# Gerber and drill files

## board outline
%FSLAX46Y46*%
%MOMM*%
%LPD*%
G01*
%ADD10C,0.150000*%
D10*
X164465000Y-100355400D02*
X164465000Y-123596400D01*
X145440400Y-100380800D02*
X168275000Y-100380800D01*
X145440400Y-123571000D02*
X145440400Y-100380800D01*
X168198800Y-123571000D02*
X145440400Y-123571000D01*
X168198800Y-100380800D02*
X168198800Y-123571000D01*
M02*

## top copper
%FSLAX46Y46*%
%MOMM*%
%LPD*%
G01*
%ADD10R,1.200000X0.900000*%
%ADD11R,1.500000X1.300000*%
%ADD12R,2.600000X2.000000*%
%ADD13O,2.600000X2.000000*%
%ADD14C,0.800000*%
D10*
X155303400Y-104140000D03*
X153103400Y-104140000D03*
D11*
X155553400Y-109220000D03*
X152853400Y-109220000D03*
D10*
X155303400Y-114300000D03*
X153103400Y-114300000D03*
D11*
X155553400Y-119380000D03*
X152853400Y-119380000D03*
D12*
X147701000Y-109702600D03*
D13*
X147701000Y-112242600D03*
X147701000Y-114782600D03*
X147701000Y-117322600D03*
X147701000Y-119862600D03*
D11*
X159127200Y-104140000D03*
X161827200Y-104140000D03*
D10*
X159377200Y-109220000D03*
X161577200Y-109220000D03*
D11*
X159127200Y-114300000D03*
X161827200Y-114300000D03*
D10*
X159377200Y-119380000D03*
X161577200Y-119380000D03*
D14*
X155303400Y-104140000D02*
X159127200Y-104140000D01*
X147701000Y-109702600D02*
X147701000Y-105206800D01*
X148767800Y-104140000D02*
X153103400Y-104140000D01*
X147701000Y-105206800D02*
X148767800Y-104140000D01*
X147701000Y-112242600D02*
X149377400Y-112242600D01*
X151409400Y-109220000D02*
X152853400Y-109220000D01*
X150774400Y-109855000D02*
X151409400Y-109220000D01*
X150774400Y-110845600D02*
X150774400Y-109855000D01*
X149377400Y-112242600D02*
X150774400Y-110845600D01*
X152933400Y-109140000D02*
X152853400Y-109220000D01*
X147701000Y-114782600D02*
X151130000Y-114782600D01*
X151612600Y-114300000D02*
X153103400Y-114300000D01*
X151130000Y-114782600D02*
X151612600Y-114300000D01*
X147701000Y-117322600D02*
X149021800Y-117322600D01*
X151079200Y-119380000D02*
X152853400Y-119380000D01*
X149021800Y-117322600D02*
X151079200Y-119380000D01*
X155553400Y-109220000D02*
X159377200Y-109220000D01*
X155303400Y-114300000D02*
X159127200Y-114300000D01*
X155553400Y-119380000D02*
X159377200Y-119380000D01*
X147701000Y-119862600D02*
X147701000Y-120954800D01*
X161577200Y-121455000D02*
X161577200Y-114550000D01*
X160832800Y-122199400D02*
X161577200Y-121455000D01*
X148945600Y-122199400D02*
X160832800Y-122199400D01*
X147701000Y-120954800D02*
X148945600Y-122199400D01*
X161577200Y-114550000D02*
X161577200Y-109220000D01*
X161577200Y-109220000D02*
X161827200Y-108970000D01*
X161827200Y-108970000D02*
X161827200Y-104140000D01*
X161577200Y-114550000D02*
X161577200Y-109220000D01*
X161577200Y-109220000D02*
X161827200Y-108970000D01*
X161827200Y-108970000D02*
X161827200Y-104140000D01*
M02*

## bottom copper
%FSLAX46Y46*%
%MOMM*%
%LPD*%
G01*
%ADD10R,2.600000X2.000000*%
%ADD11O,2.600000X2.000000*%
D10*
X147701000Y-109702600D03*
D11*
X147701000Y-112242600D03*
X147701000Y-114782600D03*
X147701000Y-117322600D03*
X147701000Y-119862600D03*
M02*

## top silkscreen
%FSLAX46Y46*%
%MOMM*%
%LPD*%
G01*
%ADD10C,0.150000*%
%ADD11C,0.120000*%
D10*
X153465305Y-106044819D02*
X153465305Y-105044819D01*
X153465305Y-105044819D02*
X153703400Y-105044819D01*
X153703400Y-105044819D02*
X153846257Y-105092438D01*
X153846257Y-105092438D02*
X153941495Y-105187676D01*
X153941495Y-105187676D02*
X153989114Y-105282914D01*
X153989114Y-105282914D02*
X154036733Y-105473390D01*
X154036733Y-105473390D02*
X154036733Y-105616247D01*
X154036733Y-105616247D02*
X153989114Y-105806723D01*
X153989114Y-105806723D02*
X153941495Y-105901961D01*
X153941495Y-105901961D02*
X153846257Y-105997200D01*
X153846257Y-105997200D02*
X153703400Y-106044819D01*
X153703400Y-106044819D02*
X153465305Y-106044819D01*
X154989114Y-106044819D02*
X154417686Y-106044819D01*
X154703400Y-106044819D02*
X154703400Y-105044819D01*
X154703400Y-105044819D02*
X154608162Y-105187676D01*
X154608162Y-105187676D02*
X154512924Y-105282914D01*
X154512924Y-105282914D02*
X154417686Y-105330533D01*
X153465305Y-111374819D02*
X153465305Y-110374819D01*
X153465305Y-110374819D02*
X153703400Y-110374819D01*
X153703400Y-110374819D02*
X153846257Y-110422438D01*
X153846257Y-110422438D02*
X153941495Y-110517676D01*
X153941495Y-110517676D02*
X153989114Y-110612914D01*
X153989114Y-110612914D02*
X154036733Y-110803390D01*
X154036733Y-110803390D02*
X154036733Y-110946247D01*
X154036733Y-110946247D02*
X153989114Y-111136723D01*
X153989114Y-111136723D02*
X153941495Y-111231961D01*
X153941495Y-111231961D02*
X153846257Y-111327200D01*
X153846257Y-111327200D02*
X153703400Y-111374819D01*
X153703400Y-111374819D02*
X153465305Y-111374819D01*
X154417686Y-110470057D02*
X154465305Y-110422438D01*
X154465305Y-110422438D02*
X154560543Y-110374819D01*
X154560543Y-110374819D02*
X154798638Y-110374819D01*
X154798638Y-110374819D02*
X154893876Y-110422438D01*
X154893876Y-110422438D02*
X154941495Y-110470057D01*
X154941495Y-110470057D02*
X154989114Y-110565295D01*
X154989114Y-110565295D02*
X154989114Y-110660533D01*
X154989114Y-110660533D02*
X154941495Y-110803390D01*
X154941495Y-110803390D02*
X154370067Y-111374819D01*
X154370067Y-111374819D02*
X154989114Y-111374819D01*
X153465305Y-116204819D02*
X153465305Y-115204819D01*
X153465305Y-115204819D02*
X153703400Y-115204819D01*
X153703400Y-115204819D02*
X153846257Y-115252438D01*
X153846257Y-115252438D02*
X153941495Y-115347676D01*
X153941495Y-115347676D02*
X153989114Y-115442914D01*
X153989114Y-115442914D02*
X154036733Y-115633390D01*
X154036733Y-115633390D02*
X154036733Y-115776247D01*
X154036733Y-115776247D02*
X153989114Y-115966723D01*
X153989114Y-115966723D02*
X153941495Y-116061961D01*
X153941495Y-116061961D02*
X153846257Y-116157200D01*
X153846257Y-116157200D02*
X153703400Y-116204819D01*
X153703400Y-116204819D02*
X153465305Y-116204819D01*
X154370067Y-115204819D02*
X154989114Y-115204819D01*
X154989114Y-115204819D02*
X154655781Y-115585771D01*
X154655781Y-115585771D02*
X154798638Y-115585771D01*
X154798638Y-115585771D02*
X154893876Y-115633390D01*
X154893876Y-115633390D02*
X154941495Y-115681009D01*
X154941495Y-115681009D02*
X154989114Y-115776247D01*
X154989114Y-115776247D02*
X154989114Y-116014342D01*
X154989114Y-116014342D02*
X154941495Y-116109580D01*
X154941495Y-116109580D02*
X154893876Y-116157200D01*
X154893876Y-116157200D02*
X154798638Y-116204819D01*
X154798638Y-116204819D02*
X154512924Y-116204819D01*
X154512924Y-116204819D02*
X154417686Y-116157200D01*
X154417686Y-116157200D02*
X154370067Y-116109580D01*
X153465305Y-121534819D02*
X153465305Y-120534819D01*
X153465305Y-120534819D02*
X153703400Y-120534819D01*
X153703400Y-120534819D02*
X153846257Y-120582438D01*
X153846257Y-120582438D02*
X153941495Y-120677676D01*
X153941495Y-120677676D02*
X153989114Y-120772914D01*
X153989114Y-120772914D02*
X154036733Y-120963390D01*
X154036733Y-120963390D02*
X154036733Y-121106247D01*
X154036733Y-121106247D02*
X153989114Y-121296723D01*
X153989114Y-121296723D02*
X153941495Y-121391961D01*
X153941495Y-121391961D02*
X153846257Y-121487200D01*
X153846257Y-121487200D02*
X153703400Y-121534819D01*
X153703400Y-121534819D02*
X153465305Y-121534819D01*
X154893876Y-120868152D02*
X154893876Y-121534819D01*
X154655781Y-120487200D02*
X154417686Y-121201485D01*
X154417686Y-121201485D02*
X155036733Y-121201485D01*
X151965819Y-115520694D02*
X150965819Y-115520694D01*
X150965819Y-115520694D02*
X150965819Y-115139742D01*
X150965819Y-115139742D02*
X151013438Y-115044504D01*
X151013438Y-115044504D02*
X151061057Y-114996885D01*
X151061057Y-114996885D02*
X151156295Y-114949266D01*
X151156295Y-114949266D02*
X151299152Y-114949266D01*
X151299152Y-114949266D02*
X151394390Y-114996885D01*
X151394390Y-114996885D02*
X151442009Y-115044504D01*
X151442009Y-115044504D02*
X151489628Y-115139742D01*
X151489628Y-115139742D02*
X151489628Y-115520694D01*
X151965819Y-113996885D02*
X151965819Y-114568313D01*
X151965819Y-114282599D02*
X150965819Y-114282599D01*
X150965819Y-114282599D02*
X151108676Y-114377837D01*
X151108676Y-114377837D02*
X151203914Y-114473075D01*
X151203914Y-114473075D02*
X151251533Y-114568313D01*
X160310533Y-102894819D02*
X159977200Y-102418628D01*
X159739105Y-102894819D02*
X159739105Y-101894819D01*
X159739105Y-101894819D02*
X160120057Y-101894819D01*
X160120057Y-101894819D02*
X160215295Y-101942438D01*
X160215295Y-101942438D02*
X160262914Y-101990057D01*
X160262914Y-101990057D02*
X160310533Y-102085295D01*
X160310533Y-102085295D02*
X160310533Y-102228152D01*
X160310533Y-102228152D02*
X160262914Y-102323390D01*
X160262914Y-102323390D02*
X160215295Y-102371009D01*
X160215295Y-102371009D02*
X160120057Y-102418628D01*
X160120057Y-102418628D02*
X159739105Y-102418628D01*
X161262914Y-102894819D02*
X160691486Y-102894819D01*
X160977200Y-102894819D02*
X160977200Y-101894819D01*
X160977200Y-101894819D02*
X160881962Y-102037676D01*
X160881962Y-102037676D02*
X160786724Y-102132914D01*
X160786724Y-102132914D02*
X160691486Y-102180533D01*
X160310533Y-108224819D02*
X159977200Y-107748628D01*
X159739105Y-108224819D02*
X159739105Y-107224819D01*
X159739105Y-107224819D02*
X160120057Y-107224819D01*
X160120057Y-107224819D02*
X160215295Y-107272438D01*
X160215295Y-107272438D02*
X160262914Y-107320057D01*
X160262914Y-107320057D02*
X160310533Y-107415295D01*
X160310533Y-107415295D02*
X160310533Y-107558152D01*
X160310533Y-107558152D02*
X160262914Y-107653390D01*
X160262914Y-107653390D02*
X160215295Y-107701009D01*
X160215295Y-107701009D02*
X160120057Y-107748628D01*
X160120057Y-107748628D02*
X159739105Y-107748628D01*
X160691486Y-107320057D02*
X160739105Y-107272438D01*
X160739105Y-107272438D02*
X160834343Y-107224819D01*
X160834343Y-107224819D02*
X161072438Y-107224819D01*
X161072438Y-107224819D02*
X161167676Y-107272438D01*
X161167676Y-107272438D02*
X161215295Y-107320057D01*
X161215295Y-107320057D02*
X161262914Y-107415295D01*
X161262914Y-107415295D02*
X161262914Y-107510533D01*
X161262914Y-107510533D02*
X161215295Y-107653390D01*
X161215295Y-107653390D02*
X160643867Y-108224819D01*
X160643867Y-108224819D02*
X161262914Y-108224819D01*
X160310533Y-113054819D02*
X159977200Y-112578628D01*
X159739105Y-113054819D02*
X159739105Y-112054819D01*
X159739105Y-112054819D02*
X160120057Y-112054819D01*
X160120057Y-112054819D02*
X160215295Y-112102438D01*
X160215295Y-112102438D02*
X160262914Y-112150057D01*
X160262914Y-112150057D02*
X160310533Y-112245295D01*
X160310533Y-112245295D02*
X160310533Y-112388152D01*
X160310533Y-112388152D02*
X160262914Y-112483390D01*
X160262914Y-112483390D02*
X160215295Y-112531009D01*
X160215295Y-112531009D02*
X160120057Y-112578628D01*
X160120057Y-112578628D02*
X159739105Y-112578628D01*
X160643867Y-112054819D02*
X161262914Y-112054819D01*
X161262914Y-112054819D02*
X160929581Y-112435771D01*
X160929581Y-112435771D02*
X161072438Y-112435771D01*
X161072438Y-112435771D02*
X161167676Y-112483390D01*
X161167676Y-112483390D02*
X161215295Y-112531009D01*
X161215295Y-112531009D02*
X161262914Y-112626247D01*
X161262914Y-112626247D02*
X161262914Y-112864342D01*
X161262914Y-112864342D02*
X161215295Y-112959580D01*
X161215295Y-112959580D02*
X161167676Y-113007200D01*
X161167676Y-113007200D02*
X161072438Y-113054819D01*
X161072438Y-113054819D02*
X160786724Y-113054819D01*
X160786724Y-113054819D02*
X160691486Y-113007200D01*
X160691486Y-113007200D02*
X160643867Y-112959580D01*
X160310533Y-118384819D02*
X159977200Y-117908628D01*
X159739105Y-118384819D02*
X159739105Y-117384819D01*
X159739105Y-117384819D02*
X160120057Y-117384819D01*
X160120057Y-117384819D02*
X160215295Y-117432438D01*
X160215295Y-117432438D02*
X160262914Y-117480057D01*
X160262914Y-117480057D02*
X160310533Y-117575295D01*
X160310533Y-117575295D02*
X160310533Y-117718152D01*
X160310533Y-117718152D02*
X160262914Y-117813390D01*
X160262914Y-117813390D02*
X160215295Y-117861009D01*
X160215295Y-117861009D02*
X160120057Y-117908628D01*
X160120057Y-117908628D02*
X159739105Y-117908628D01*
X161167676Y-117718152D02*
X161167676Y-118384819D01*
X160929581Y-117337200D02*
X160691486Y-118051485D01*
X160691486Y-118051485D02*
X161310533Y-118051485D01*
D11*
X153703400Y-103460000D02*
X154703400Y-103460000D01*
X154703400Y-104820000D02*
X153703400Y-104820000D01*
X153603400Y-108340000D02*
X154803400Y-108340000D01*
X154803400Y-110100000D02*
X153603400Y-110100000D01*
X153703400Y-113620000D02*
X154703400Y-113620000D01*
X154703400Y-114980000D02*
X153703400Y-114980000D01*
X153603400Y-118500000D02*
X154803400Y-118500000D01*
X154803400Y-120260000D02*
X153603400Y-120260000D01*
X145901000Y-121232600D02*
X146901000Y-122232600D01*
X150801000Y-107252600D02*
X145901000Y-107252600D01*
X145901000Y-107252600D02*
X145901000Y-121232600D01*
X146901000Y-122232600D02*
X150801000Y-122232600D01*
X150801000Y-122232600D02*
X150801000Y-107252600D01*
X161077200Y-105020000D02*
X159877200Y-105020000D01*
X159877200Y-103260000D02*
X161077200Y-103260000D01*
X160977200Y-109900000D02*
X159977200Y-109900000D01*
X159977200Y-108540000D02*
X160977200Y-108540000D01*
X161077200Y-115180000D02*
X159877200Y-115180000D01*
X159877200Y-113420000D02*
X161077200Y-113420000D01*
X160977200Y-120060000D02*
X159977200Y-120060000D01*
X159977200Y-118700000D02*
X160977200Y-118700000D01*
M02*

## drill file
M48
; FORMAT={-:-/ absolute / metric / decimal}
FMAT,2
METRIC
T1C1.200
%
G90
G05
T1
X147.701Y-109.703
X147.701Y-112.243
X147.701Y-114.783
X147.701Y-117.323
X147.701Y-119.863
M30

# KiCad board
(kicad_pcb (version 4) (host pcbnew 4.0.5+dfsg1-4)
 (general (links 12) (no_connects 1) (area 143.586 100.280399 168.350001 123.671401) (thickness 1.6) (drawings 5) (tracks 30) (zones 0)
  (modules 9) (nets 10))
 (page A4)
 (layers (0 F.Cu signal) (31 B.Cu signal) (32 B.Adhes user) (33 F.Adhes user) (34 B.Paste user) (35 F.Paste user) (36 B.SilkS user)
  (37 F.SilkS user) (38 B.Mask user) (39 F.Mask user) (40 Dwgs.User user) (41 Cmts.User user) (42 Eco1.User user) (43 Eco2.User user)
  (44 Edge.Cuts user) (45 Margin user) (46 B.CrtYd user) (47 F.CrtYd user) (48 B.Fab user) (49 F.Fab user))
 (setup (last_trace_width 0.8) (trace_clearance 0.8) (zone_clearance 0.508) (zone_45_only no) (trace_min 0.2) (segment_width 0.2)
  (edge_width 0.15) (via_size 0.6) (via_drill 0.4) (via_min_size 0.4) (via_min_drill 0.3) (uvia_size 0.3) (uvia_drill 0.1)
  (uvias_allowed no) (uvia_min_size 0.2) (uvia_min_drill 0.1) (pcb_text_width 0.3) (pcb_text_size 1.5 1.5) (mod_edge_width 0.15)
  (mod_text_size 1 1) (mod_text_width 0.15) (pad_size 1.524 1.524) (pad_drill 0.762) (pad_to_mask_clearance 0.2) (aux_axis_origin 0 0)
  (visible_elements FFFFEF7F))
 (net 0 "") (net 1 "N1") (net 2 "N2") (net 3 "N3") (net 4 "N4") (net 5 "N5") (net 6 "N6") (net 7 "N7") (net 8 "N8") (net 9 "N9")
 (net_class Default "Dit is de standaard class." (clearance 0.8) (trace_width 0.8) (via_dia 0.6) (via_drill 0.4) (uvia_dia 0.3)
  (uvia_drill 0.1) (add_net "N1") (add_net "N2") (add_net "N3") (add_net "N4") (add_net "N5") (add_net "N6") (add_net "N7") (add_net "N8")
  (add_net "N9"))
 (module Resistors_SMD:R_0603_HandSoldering (layer F.Cu) (at 154.2034 104.14 180)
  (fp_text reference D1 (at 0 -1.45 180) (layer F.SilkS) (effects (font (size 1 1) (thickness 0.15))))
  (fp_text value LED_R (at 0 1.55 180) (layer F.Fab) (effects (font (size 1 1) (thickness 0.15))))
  (fp_line (start 0.5 0.68) (end -0.5 0.68) (layer F.SilkS) (width 0.12))
  (fp_line (start -0.5 -0.68) (end 0.5 -0.68) (layer F.SilkS) (width 0.12))
  (pad 1 smd rect (at -1.1 0 180) (size 1.2 0.9) (layers F.Cu F.Paste F.Mask) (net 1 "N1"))
  (pad 2 smd rect (at 1.1 0 180) (size 1.2 0.9) (layers F.Cu F.Paste F.Mask) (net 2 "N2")))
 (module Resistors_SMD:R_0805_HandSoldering (layer F.Cu) (at 154.2034 109.22 180)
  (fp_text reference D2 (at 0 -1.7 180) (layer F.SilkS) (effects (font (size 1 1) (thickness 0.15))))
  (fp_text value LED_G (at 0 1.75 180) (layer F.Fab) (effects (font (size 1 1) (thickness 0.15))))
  (fp_line (start 0.6 0.88) (end -0.6 0.88) (layer F.SilkS) (width 0.12))
  (fp_line (start -0.6 -0.88) (end 0.6 -0.88) (layer F.SilkS) (width 0.12))
  (pad 1 smd rect (at -1.35 0 180) (size 1.5 1.3) (layers F.Cu F.Paste F.Mask) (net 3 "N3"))
  (pad 2 smd rect (at 1.35 0 180) (size 1.5 1.3) (layers F.Cu F.Paste F.Mask) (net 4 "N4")))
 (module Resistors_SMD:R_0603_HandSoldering (layer F.Cu) (at 154.2034 114.3 180)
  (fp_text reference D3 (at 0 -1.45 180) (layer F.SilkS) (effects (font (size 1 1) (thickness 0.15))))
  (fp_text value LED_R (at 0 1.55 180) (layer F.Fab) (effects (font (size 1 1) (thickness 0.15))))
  (fp_line (start 0.5 0.68) (end -0.5 0.68) (layer F.SilkS) (width 0.12))
  (fp_line (start -0.5 -0.68) (end 0.5 -0.68) (layer F.SilkS) (width 0.12))
  (pad 1 smd rect (at -1.1 0 180) (size 1.2 0.9) (layers F.Cu F.Paste F.Mask) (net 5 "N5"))
  (pad 2 smd rect (at 1.1 0 180) (size 1.2 0.9) (layers F.Cu F.Paste F.Mask) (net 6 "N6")))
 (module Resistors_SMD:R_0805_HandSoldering (layer F.Cu) (at 154.2034 119.38 180)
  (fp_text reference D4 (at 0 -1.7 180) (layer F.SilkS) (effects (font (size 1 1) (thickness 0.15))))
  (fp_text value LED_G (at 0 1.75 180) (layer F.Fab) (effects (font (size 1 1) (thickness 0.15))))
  (fp_line (start 0.6 0.88) (end -0.6 0.88) (layer F.SilkS) (width 0.12))
  (fp_line (start -0.6 -0.88) (end 0.6 -0.88) (layer F.SilkS) (width 0.12))
  (pad 1 smd rect (at -1.35 0 180) (size 1.5 1.3) (layers F.Cu F.Paste F.Mask) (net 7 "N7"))
  (pad 2 smd rect (at 1.35 0 180) (size 1.5 1.3) (layers F.Cu F.Paste F.Mask) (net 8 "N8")))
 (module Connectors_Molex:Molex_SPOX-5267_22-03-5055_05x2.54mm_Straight (layer F.Cu) (at 147.701 109.7026 270)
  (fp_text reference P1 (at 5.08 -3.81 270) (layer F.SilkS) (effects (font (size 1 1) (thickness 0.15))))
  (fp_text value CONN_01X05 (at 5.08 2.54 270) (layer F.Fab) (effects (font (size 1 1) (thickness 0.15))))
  (fp_line (start 11.53 1.8) (end 12.53 0.8) (layer F.SilkS) (width 0.12))
  (fp_line (start -2.45 -3.1) (end -2.45 1.8) (layer F.SilkS) (width 0.12))
  (fp_line (start -2.45 1.8) (end 11.53 1.8) (layer F.SilkS) (width 0.12))
  (fp_line (start 12.53 0.8) (end 12.53 -3.1) (layer F.SilkS) (width 0.12))
  (fp_line (start 12.53 -3.1) (end -2.45 -3.1) (layer F.SilkS) (width 0.12))
  (pad 1 thru_hole rect (at 0 0 270) (size 2 2.6) (drill 1.2) (layers *.Cu *.Mask) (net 2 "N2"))
  (pad 2 thru_hole oval (at 2.54 0 270) (size 2 2.6) (drill 1.2) (layers *.Cu *.Mask) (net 4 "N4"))
  (pad 3 thru_hole oval (at 5.08 0 270) (size 2 2.6) (drill 1.2) (layers *.Cu *.Mask) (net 6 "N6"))
  (pad 4 thru_hole oval (at 7.62 0 270) (size 2 2.6) (drill 1.2) (layers *.Cu *.Mask) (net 8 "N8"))
  (pad 5 thru_hole oval (at 10.16 0 270) (size 2 2.6) (drill 1.2) (layers *.Cu *.Mask) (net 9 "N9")))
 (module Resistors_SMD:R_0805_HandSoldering (layer F.Cu) (at 160.4772 104.14)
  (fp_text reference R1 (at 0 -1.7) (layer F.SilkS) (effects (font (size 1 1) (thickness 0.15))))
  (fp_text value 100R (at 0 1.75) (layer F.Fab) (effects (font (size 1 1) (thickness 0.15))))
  (fp_line (start 0.6 0.88) (end -0.6 0.88) (layer F.SilkS) (width 0.12))
  (fp_line (start -0.6 -0.88) (end 0.6 -0.88) (layer F.SilkS) (width 0.12))
  (pad 1 smd rect (at -1.35 0) (size 1.5 1.3) (layers F.Cu F.Paste F.Mask) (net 1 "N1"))
  (pad 2 smd rect (at 1.35 0) (size 1.5 1.3) (layers F.Cu F.Paste F.Mask) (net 9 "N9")))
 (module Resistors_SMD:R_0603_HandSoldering (layer F.Cu) (at 160.4772 109.22)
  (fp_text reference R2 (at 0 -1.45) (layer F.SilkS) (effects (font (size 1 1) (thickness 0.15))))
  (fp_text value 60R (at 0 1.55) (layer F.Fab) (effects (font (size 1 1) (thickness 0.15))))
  (fp_line (start 0.5 0.68) (end -0.5 0.68) (layer F.SilkS) (width 0.12))
  (fp_line (start -0.5 -0.68) (end 0.5 -0.68) (layer F.SilkS) (width 0.12))
  (pad 1 smd rect (at -1.1 0) (size 1.2 0.9) (layers F.Cu F.Paste F.Mask) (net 3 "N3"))
  (pad 2 smd rect (at 1.1 0) (size 1.2 0.9) (layers F.Cu F.Paste F.Mask) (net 9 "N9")))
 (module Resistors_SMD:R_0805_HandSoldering (layer F.Cu) (at 160.4772 114.3)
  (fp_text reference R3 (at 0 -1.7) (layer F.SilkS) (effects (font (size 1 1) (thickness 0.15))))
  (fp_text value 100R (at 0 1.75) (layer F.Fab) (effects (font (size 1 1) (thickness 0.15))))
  (fp_line (start 0.6 0.88) (end -0.6 0.88) (layer F.SilkS) (width 0.12))
  (fp_line (start -0.6 -0.88) (end 0.6 -0.88) (layer F.SilkS) (width 0.12))
  (pad 1 smd rect (at -1.35 0) (size 1.5 1.3) (layers F.Cu F.Paste F.Mask) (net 5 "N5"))
  (pad 2 smd rect (at 1.35 0) (size 1.5 1.3) (layers F.Cu F.Paste F.Mask) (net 9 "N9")))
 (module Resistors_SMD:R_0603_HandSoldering (layer F.Cu) (at 160.4772 119.38)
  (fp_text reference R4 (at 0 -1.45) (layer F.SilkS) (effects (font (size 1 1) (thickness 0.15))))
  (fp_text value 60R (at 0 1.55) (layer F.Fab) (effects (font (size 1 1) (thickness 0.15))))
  (fp_line (start 0.5 0.68) (end -0.5 0.68) (layer F.SilkS) (width 0.12))
  (fp_line (start -0.5 -0.68) (end 0.5 -0.68) (layer F.SilkS) (width 0.12))
  (pad 1 smd rect (at -1.1 0) (size 1.2 0.9) (layers F.Cu F.Paste F.Mask) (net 7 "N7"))
  (pad 2 smd rect (at 1.1 0) (size 1.2 0.9) (layers F.Cu F.Paste F.Mask) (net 9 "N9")))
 (gr_line (start 164.465 100.3554) (end 164.465 123.5964) (angle 90) (layer Edge.Cuts) (width 0.15))
 (gr_line (start 145.4404 100.3808) (end 168.275 100.3808) (angle 90) (layer Edge.Cuts) (width 0.15))
 (gr_line (start 145.4404 123.571) (end 145.4404 100.3808) (angle 90) (layer Edge.Cuts) (width 0.15))
 (gr_line (start 168.1988 123.571) (end 145.4404 123.571) (angle 90) (layer Edge.Cuts) (width 0.15))
 (gr_line (start 168.1988 100.3808) (end 168.1988 123.571) (angle 90) (layer Edge.Cuts) (width 0.15))
 (segment (start 155.3034 104.14) (end 159.1272 104.14) (width 0.8) (layer F.Cu) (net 1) (status C00000))
 (segment (start 147.701 109.7026) (end 147.701 105.2068) (width 0.8) (layer F.Cu) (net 2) (status 400000))
 (segment (start 148.7678 104.14) (end 153.1034 104.14) (width 0.8) (layer F.Cu) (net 2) (status 800000))
 (segment (start 147.701 105.2068) (end 148.7678 104.14) (width 0.8) (layer F.Cu) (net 2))
 (segment (start 147.701 112.2426) (end 149.3774 112.2426) (width 0.8) (layer F.Cu) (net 4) (status 400000))
 (segment (start 151.4094 109.22) (end 152.8534 109.22) (width 0.8) (layer F.Cu) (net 4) (status 800000))
 (segment (start 150.7744 109.855) (end 151.4094 109.22) (width 0.8) (layer F.Cu) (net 4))
 (segment (start 150.7744 110.8456) (end 150.7744 109.855) (width 0.8) (layer F.Cu) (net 4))
 (segment (start 149.3774 112.2426) (end 150.7744 110.8456) (width 0.8) (layer F.Cu) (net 4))
 (segment (start 152.9334 109.14) (end 152.8534 109.22) (width 0.8) (layer F.Cu) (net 4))
 (segment (start 147.701 114.7826) (end 151.13 114.7826) (width 0.8) (layer F.Cu) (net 6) (status 400000))
 (segment (start 151.6126 114.3) (end 153.1034 114.3) (width 0.8) (layer F.Cu) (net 6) (status 800000))
 (segment (start 151.13 114.7826) (end 151.6126 114.3) (width 0.8) (layer F.Cu) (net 6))
 (segment (start 147.701 117.3226) (end 149.0218 117.3226) (width 0.8) (layer F.Cu) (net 8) (status 400000))
 (segment (start 151.0792 119.38) (end 152.8534 119.38) (width 0.8) (layer F.Cu) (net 8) (status 800000))
 (segment (start 149.0218 117.3226) (end 151.0792 119.38) (width 0.8) (layer F.Cu) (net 8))
 (segment (start 155.5534 109.22) (end 159.3772 109.22) (width 0.8) (layer F.Cu) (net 3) (status C00000))
 (segment (start 155.3034 114.3) (end 159.1272 114.3) (width 0.8) (layer F.Cu) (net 5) (status C00000))
 (segment (start 155.5534 119.38) (end 159.3772 119.38) (width 0.8) (layer F.Cu) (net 7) (status C00000))
 (segment (start 147.701 119.8626) (end 147.701 120.9548) (width 0.8) (layer F.Cu) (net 9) (status 400000))
 (segment (start 161.5772 121.455) (end 161.5772 114.55) (width 0.8) (layer F.Cu) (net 9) (status 800000))
 (segment (start 160.8328 122.1994) (end 161.5772 121.455) (width 0.8) (layer F.Cu) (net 9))
 (segment (start 148.9456 122.1994) (end 160.8328 122.1994) (width 0.8) (layer F.Cu) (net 9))
 (segment (start 147.701 120.9548) (end 148.9456 122.1994) (width 0.8) (layer F.Cu) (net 9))
 (segment (start 161.5772 114.55) (end 161.5772 109.22) (width 0.8) (layer F.Cu) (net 9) (status C00000))
 (segment (start 161.5772 109.22) (end 161.8272 108.97) (width 0.8) (layer F.Cu) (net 9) (status C00000))
 (segment (start 161.8272 108.97) (end 161.8272 104.14) (width 0.8) (layer F.Cu) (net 9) (status C00000))
 (segment (start 161.5772 114.55) (end 161.5772 109.22) (width 0.8) (layer F.Cu) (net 9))
 (segment (start 161.5772 109.22) (end 161.8272 108.97) (width 0.8) (layer F.Cu) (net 9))
 (segment (start 161.8272 108.97) (end 161.8272 104.14) (width 0.8) (layer F.Cu) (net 9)))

